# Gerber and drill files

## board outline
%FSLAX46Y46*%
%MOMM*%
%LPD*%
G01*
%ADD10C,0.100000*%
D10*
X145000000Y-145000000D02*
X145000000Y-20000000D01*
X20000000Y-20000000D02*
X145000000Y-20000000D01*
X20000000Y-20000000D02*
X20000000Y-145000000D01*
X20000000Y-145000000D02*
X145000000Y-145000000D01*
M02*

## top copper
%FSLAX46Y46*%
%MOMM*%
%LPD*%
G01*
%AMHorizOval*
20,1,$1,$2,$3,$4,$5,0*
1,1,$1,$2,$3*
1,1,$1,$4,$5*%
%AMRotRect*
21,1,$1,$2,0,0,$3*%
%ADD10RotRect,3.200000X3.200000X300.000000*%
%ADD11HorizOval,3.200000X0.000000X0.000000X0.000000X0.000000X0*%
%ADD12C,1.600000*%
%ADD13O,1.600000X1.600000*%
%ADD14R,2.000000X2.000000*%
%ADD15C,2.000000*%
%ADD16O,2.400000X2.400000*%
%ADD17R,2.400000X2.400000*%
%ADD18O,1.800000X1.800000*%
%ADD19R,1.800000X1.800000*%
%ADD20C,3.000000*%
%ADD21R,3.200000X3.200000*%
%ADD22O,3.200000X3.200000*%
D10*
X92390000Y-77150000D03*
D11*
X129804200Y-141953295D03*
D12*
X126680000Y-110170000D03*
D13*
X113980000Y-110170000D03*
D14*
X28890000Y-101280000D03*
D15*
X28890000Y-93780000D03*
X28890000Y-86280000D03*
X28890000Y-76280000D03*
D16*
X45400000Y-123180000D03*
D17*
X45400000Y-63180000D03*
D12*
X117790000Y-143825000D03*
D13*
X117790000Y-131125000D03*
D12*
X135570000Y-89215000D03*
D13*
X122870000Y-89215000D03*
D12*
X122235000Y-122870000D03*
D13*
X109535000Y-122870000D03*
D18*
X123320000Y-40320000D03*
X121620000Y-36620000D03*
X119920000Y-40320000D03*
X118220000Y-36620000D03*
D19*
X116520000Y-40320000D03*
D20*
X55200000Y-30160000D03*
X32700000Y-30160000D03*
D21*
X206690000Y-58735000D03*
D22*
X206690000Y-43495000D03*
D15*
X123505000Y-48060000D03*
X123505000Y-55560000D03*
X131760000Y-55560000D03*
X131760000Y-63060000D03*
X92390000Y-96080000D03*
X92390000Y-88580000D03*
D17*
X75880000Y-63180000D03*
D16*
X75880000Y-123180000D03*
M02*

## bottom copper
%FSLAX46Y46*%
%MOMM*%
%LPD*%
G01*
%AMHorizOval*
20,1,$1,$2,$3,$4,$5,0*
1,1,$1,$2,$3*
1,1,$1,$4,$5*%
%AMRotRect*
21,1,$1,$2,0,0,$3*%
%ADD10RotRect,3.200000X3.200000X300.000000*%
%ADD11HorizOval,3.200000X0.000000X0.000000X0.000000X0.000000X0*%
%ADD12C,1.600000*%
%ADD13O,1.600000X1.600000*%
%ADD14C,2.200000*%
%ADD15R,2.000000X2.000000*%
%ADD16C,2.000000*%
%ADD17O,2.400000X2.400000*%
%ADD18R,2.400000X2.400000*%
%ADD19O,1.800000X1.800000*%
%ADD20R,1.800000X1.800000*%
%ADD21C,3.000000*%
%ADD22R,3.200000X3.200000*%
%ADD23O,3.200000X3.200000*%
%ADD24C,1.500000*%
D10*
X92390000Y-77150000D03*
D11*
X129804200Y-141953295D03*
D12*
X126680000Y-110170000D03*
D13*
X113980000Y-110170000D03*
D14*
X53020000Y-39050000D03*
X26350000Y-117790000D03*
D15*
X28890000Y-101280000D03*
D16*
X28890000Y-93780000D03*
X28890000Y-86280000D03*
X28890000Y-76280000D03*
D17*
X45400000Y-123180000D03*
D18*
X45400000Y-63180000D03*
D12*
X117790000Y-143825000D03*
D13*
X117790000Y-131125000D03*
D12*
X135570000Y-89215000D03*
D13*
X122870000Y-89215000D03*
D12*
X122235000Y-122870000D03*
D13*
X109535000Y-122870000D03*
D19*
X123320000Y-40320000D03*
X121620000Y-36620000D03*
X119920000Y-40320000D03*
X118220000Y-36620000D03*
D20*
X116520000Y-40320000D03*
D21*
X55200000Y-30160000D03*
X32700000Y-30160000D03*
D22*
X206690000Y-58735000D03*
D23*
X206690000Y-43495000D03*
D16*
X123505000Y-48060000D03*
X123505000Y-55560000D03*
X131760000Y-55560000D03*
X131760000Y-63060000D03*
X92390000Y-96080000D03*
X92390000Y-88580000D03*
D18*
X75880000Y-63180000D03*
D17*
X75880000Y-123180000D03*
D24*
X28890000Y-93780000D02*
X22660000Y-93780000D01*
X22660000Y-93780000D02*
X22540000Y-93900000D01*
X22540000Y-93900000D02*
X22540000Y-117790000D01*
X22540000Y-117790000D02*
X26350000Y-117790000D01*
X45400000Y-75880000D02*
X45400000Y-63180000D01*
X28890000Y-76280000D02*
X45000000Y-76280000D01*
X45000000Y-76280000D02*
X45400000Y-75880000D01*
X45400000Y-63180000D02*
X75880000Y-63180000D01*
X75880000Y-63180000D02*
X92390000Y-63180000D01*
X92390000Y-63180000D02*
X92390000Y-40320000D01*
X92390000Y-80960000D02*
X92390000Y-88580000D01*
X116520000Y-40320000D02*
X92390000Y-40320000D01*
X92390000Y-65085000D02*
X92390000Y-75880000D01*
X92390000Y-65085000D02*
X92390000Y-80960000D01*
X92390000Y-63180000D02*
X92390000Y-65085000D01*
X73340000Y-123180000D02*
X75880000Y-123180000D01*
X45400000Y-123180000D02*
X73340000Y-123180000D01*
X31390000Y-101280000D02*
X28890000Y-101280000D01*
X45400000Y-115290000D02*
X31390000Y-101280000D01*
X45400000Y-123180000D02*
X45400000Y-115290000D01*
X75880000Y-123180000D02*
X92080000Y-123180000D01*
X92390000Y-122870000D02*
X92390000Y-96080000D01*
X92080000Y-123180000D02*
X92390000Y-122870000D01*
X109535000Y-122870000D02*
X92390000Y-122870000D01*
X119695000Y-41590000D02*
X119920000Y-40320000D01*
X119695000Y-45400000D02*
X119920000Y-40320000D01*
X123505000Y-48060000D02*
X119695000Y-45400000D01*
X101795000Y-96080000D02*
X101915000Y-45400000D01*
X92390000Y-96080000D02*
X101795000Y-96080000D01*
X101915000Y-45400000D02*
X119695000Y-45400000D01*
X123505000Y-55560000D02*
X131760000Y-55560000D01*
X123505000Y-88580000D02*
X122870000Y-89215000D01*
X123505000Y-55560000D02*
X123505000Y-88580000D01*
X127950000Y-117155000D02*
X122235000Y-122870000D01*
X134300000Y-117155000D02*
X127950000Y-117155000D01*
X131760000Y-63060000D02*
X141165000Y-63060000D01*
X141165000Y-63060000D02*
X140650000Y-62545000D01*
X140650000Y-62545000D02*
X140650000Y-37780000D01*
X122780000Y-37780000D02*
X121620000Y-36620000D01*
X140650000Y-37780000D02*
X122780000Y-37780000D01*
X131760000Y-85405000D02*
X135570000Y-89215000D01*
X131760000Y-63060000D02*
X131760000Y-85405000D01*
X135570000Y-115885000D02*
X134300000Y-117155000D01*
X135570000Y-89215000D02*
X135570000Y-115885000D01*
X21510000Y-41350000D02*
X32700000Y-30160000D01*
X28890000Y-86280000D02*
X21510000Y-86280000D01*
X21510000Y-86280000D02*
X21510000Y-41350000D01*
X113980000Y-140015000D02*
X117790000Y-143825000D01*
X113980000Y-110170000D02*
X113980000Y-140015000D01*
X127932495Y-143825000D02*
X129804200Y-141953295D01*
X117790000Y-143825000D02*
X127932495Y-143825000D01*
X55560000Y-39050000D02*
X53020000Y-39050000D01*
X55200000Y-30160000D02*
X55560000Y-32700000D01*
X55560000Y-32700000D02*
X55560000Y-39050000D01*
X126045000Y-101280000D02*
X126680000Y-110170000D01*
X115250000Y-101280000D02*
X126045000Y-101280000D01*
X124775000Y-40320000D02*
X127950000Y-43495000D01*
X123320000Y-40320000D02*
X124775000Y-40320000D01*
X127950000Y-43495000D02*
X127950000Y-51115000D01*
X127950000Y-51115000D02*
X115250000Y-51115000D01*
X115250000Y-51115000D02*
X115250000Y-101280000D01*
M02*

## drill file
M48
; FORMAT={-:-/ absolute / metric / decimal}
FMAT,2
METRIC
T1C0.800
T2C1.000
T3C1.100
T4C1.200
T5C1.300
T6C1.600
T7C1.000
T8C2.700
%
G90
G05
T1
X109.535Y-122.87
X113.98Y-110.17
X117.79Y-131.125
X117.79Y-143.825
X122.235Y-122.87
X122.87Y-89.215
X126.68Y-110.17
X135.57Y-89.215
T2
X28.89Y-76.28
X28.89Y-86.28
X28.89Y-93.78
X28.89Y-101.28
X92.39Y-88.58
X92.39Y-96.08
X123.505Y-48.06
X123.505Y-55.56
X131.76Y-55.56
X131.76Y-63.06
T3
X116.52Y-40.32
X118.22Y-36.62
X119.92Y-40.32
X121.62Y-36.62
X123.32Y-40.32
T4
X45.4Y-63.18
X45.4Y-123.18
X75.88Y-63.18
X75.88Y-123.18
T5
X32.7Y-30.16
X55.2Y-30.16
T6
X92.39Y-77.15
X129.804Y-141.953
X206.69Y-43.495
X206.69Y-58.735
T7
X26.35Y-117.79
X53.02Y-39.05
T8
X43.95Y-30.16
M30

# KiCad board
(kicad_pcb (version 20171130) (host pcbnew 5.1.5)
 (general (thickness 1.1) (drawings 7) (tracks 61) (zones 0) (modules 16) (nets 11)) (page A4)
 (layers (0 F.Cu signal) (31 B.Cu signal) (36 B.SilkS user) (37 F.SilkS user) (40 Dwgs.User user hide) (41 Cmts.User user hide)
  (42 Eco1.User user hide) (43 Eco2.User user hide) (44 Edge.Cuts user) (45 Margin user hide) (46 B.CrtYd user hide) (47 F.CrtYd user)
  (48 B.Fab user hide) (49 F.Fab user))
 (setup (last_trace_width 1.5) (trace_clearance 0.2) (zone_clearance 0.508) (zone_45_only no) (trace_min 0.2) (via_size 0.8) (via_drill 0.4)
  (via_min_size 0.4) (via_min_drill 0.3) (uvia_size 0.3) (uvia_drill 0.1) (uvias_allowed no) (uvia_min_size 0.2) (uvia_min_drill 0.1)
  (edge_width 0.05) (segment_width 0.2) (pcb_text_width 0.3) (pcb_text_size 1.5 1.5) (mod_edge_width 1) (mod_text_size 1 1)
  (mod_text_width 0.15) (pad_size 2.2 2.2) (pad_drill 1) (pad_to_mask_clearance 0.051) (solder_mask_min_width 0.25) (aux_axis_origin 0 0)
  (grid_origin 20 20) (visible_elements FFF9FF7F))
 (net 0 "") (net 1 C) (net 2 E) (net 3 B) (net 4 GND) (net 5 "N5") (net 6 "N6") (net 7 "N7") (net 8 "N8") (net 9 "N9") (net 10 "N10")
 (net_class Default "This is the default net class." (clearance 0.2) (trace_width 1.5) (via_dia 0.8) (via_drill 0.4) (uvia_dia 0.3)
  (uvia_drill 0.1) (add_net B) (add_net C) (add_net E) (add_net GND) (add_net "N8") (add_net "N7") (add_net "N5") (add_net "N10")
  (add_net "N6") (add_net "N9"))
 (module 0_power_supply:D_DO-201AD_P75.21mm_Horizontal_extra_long (layer B.Cu) (at 92.39 77.15 300)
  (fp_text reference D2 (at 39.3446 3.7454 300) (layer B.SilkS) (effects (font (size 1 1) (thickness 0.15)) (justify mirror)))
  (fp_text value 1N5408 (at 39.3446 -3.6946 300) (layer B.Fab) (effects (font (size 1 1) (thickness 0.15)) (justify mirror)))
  (pad 1 thru_hole rect (at 0 0 300) (size 3.2 3.2) (drill 1.6) (layers *.Cu *.Mask) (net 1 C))
  (pad 2 thru_hole oval (at 74.8284 0 300) (size 3.2 3.2) (drill 1.6) (layers *.Cu *.Mask) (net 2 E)))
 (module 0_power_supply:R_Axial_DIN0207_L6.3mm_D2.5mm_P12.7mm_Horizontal (layer F.Cu) (at 126.68 110.17 180)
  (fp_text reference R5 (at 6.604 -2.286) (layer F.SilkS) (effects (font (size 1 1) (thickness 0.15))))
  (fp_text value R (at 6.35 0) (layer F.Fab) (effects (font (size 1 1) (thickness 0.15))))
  (pad 1 thru_hole circle (at 0 0 180) (size 1.6 1.6) (drill 0.8) (layers *.Cu *.Mask) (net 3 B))
  (pad 2 thru_hole oval (at 12.7 0 180) (size 1.6 1.6) (drill 0.8) (layers *.Cu *.Mask) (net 2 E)))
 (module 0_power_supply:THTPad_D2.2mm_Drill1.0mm (layer B.Cu) (at 53.02 39.05)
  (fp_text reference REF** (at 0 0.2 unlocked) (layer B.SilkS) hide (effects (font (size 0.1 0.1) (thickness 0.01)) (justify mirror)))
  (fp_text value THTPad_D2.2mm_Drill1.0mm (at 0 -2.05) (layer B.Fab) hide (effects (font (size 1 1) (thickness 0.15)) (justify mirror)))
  (pad "" np_thru_hole circle (at 0 0) (size 2.2 2.2) (drill 1) (layers B.Cu)))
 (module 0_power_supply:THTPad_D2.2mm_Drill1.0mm (layer B.Cu) (at 26.35 117.79)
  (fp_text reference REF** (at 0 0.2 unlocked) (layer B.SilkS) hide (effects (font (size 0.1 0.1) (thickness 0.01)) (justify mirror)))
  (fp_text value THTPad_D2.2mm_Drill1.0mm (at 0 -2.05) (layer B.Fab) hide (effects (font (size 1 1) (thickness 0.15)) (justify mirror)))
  (pad "" np_thru_hole circle (at 0 0) (size 2.2 2.2) (drill 1) (layers B.Cu)))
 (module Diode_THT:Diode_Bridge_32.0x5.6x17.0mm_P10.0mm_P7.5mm (layer F.Cu) (at 28.89 101.28 90)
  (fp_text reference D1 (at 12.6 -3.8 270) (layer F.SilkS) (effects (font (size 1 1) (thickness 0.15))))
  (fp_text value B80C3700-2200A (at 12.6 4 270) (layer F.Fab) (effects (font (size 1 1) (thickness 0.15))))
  (pad 1 thru_hole rect (at 0 0 90) (size 2 2) (drill 1) (layers *.Cu *.Mask) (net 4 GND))
  (pad 2 thru_hole circle (at 7.5 0 90) (size 2 2) (drill 1) (layers *.Cu *.Mask))
  (pad 3 thru_hole circle (at 15 0 90) (size 2 2) (drill 1) (layers *.Cu *.Mask) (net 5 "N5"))
  (pad 4 thru_hole circle (at 25 0 90) (size 2 2) (drill 1) (layers *.Cu *.Mask) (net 1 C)))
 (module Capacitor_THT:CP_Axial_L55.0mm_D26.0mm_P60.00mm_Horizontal (layer F.Cu) (at 45.4 63.18 270)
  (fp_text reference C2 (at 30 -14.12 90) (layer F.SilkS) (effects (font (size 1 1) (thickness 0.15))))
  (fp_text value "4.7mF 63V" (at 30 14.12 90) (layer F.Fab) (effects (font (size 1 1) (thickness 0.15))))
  (pad 2 thru_hole oval (at 60 0 270) (size 2.4 2.4) (drill 1.2) (layers *.Cu *.Mask) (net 4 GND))
  (pad 1 thru_hole rect (at 0 0 270) (size 2.4 2.4) (drill 1.2) (layers *.Cu *.Mask) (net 1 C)))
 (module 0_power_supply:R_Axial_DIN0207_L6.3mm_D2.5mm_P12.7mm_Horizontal (layer F.Cu) (at 117.79 143.825 90)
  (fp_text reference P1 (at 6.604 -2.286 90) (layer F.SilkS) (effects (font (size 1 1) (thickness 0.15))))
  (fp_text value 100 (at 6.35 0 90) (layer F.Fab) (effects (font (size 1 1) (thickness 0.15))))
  (pad 1 thru_hole circle (at 0 0 90) (size 1.6 1.6) (drill 0.8) (layers *.Cu *.Mask) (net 2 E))
  (pad 2 thru_hole oval (at 12.7 0 90) (size 1.6 1.6) (drill 0.8) (layers *.Cu *.Mask) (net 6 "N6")))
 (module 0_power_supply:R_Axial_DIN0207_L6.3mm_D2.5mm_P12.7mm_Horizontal (layer F.Cu) (at 135.57 89.215 180)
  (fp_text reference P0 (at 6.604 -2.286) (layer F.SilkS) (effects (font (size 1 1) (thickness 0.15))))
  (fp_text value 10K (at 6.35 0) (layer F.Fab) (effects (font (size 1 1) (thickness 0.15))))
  (pad 1 thru_hole circle (at 0 0 180) (size 1.6 1.6) (drill 0.8) (layers *.Cu *.Mask) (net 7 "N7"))
  (pad 2 thru_hole oval (at 12.7 0 180) (size 1.6 1.6) (drill 0.8) (layers *.Cu *.Mask) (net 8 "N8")))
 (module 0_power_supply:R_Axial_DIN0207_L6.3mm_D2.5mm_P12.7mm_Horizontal (layer F.Cu) (at 122.235 122.87 180)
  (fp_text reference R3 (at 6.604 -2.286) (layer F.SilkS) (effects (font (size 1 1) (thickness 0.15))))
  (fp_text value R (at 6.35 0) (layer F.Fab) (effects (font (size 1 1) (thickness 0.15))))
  (pad 1 thru_hole circle (at 0 0 180) (size 1.6 1.6) (drill 0.8) (layers *.Cu *.Mask) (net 7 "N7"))
  (pad 2 thru_hole oval (at 12.7 0 180) (size 1.6 1.6) (drill 0.8) (layers *.Cu *.Mask) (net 4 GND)))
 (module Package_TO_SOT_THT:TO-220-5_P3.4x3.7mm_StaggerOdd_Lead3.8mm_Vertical (layer F.Cu) (at 116.52 40.32)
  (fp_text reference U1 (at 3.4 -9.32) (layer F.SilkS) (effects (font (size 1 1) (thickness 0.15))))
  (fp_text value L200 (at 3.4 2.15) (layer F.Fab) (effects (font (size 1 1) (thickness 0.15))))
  (pad 5 thru_hole oval (at 6.8 0) (size 1.8 1.8) (drill 1.1) (layers *.Cu *.Mask) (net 3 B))
  (pad 4 thru_hole oval (at 5.1 -3.7) (size 1.8 1.8) (drill 1.1) (layers *.Cu *.Mask) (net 7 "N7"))
  (pad 3 thru_hole oval (at 3.4 0) (size 1.8 1.8) (drill 1.1) (layers *.Cu *.Mask) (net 4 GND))
  (pad 2 thru_hole oval (at 1.7 -3.7) (size 1.8 1.8) (drill 1.1) (layers *.Cu *.Mask) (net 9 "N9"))
  (pad 1 thru_hole rect (at 0 0) (size 1.8 1.8) (drill 1.1) (layers *.Cu *.Mask) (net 1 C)))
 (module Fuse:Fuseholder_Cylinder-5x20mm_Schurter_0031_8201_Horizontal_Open (layer F.Cu) (at 32.7 30.16)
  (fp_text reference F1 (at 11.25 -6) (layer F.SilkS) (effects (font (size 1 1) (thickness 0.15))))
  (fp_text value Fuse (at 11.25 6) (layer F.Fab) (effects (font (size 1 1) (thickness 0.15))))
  (pad "" np_thru_hole circle (at 11.25 0) (size 2.7 2.7) (drill 2.7) (layers *.Cu *.Mask))
  (pad 2 thru_hole circle (at 22.5 0) (size 3 3) (drill 1.3) (layers *.Cu *.Mask) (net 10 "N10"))
  (pad 1 thru_hole circle (at 0 0) (size 3 3) (drill 1.3) (layers *.Cu *.Mask) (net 5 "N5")))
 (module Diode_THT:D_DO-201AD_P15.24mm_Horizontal (layer B.Cu) (at 206.69 58.735 90)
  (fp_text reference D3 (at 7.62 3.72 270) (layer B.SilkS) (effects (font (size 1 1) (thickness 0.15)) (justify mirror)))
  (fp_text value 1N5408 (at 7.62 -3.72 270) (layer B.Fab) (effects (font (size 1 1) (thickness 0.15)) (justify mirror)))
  (pad 1 thru_hole rect (at 0 0 90) (size 3.2 3.2) (drill 1.6) (layers *.Cu *.Mask) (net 8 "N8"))
  (pad 2 thru_hole oval (at 15.24 0 90) (size 3.2 3.2) (drill 1.6) (layers *.Cu *.Mask) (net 4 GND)))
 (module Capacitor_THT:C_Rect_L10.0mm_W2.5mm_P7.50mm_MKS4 (layer F.Cu) (at 123.505 55.56 90)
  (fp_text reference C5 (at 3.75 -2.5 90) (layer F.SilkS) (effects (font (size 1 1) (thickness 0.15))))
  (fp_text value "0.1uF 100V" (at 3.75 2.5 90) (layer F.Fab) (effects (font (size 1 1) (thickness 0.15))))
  (pad 2 thru_hole circle (at 7.5 0 90) (size 2 2) (drill 1) (layers *.Cu *.Mask) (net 4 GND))
  (pad 1 thru_hole circle (at 0 0 90) (size 2 2) (drill 1) (layers *.Cu *.Mask) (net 8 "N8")))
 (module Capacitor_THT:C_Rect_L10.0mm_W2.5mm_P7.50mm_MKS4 (layer F.Cu) (at 131.76 55.56 270)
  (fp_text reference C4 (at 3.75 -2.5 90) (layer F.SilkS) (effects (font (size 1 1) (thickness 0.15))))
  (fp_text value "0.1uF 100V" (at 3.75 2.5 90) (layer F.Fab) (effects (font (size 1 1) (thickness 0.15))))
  (pad 1 thru_hole circle (at 0 0 270) (size 2 2) (drill 1) (layers *.Cu *.Mask) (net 8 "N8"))
  (pad 2 thru_hole circle (at 7.5 0 270) (size 2 2) (drill 1) (layers *.Cu *.Mask) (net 7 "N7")))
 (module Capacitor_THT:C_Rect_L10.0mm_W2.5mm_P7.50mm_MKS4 (layer F.Cu) (at 92.39 88.58 270)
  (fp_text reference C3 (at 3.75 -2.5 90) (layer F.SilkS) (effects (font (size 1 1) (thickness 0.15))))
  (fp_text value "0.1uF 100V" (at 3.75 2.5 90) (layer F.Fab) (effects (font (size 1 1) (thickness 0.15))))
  (pad 2 thru_hole circle (at 7.5 0 270) (size 2 2) (drill 1) (layers *.Cu *.Mask) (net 4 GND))
  (pad 1 thru_hole circle (at 0 0 270) (size 2 2) (drill 1) (layers *.Cu *.Mask) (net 1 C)))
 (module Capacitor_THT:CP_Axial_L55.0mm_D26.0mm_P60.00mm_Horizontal (layer F.Cu) (at 75.88 63.18 270)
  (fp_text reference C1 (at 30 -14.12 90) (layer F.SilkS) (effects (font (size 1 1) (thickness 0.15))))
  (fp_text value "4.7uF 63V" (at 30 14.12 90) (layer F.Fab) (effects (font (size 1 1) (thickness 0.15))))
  (pad 1 thru_hole rect (at 0 0 270) (size 2.4 2.4) (drill 1.2) (layers *.Cu *.Mask) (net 1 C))
  (pad 2 thru_hole oval (at 60 0 270) (size 2.4 2.4) (drill 1.2) (layers *.Cu *.Mask) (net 4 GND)))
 (gr_line (start 145 145) (end 145 20) (layer Edge.Cuts) (width 0.1))
 (gr_line (start 20 20) (end 145 20) (layer Edge.Cuts) (width 0.1))
 (gr_line (start 20 20) (end 20 145) (layer Edge.Cuts) (width 0.1))
 (gr_line (start 20 145) (end 145 145) (layer Edge.Cuts) (width 0.1))
 (segment (start 28.89 93.78) (end 22.66 93.78) (width 1.5) (layer B.Cu) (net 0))
 (segment (start 22.66 93.78) (end 22.54 93.9) (width 1.5) (layer B.Cu) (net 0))
 (segment (start 22.54 93.9) (end 22.54 117.79) (width 1.5) (layer B.Cu) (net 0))
 (segment (start 22.54 117.79) (end 26.35 117.79) (width 1.5) (layer B.Cu) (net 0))
 (segment (start 45.4 75.88) (end 45.4 63.18) (width 1.5) (layer B.Cu) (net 1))
 (segment (start 28.89 76.28) (end 45 76.28) (width 1.5) (layer B.Cu) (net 1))
 (segment (start 45 76.28) (end 45.4 75.88) (width 1.5) (layer B.Cu) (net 1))
 (segment (start 45.4 63.18) (end 75.88 63.18) (width 1.5) (layer B.Cu) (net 1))
 (segment (start 75.88 63.18) (end 92.39 63.18) (width 1.5) (layer B.Cu) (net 1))
 (segment (start 92.39 63.18) (end 92.39 40.32) (width 1.5) (layer B.Cu) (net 1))
 (segment (start 92.39 80.96) (end 92.39 88.58) (width 1.5) (layer B.Cu) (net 1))
 (segment (start 116.52 40.32) (end 92.39 40.32) (width 1.5) (layer B.Cu) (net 1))
 (segment (start 92.39 65.085) (end 92.39 75.88) (width 1.5) (layer B.Cu) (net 1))
 (segment (start 92.39 65.085) (end 92.39 80.96) (width 1.5) (layer B.Cu) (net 1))
 (segment (start 92.39 63.18) (end 92.39 65.085) (width 1.5) (layer B.Cu) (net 1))
 (segment (start 73.34 123.18) (end 75.88 123.18) (width 1.5) (layer B.Cu) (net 4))
 (segment (start 45.4 123.18) (end 73.34 123.18) (width 1.5) (layer B.Cu) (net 4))
 (segment (start 31.39 101.28) (end 28.89 101.28) (width 1.5) (layer B.Cu) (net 4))
 (segment (start 45.4 115.29) (end 31.39 101.28) (width 1.5) (layer B.Cu) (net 4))
 (segment (start 45.4 123.18) (end 45.4 115.29) (width 1.5) (layer B.Cu) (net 4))
 (segment (start 75.88 123.18) (end 92.08 123.18) (width 1.5) (layer B.Cu) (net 4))
 (segment (start 92.39 122.87) (end 92.39 96.08) (width 1.5) (layer B.Cu) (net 4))
 (segment (start 92.08 123.18) (end 92.39 122.87) (width 1.5) (layer B.Cu) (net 4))
 (segment (start 109.535 122.87) (end 92.39 122.87) (width 1.5) (layer B.Cu) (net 4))
 (segment (start 119.695 41.59) (end 119.92 40.32) (width 1.5) (layer B.Cu) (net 4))
 (segment (start 119.695 45.4) (end 119.92 40.32) (width 1.5) (layer B.Cu) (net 4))
 (segment (start 123.505 48.06) (end 119.695 45.4) (width 1.5) (layer B.Cu) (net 4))
 (segment (start 101.795 96.08) (end 101.915 45.4) (width 1.5) (layer B.Cu) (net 4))
 (segment (start 92.39 96.08) (end 101.795 96.08) (width 1.5) (layer B.Cu) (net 4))
 (segment (start 101.915 45.4) (end 119.695 45.4) (width 1.5) (layer B.Cu) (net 4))
 (segment (start 123.505 55.56) (end 131.76 55.56) (width 1.5) (layer B.Cu) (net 8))
 (segment (start 123.505 88.58) (end 122.87 89.215) (width 1.5) (layer B.Cu) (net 8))
 (segment (start 123.505 55.56) (end 123.505 88.58) (width 1.5) (layer B.Cu) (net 8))
 (segment (start 127.95 117.155) (end 122.235 122.87) (width 1.5) (layer B.Cu) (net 7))
 (segment (start 134.3 117.155) (end 127.95 117.155) (width 1.5) (layer B.Cu) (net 7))
 (segment (start 131.76 63.06) (end 141.165 63.06) (width 1.5) (layer B.Cu) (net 7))
 (segment (start 141.165 63.06) (end 140.65 62.545) (width 1.5) (layer B.Cu) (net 7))
 (segment (start 140.65 62.545) (end 140.65 37.78) (width 1.5) (layer B.Cu) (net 7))
 (segment (start 122.78 37.78) (end 121.62 36.62) (width 1.5) (layer B.Cu) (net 7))
 (segment (start 140.65 37.78) (end 122.78 37.78) (width 1.5) (layer B.Cu) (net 7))
 (segment (start 131.76 85.405) (end 135.57 89.215) (width 1.5) (layer B.Cu) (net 7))
 (segment (start 131.76 63.06) (end 131.76 85.405) (width 1.5) (layer B.Cu) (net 7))
 (segment (start 135.57 115.885) (end 134.3 117.155) (width 1.5) (layer B.Cu) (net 7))
 (segment (start 135.57 89.215) (end 135.57 115.885) (width 1.5) (layer B.Cu) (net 7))
 (segment (start 21.51 41.35) (end 32.7 30.16) (width 1.5) (layer B.Cu) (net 5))
 (segment (start 28.89 86.28) (end 21.51 86.28) (width 1.5) (layer B.Cu) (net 5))
 (segment (start 21.51 86.28) (end 21.51 41.35) (width 1.5) (layer B.Cu) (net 5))
 (segment (start 113.98 140.015) (end 117.79 143.825) (width 1.5) (layer B.Cu) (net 2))
 (segment (start 113.98 110.17) (end 113.98 140.015) (width 1.5) (layer B.Cu) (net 2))
 (segment (start 127.932495 143.825) (end 129.8042 141.953295) (width 1.5) (layer B.Cu) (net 2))
 (segment (start 117.79 143.825) (end 127.932495 143.825) (width 1.5) (layer B.Cu) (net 2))
 (segment (start 55.56 39.05) (end 53.02 39.05) (width 1.5) (layer B.Cu) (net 10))
 (segment (start 55.2 30.16) (end 55.56 32.7) (width 1.5) (layer B.Cu) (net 10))
 (segment (start 55.56 32.7) (end 55.56 39.05) (width 1.5) (layer B.Cu) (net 10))
 (segment (start 126.045 101.28) (end 126.68 110.17) (width 1.5) (layer B.Cu) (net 3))
 (segment (start 115.25 101.28) (end 126.045 101.28) (width 1.5) (layer B.Cu) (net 3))
 (segment (start 124.775 40.32) (end 127.95 43.495) (width 1.5) (layer B.Cu) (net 3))
 (segment (start 123.32 40.32) (end 124.775 40.32) (width 1.5) (layer B.Cu) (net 3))
 (segment (start 127.95 43.495) (end 127.95 51.115) (width 1.5) (layer B.Cu) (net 3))
 (segment (start 127.95 51.115) (end 115.25 51.115) (width 1.5) (layer B.Cu) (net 3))
 (segment (start 115.25 51.115) (end 115.25 101.28) (width 1.5) (layer B.Cu) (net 3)))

